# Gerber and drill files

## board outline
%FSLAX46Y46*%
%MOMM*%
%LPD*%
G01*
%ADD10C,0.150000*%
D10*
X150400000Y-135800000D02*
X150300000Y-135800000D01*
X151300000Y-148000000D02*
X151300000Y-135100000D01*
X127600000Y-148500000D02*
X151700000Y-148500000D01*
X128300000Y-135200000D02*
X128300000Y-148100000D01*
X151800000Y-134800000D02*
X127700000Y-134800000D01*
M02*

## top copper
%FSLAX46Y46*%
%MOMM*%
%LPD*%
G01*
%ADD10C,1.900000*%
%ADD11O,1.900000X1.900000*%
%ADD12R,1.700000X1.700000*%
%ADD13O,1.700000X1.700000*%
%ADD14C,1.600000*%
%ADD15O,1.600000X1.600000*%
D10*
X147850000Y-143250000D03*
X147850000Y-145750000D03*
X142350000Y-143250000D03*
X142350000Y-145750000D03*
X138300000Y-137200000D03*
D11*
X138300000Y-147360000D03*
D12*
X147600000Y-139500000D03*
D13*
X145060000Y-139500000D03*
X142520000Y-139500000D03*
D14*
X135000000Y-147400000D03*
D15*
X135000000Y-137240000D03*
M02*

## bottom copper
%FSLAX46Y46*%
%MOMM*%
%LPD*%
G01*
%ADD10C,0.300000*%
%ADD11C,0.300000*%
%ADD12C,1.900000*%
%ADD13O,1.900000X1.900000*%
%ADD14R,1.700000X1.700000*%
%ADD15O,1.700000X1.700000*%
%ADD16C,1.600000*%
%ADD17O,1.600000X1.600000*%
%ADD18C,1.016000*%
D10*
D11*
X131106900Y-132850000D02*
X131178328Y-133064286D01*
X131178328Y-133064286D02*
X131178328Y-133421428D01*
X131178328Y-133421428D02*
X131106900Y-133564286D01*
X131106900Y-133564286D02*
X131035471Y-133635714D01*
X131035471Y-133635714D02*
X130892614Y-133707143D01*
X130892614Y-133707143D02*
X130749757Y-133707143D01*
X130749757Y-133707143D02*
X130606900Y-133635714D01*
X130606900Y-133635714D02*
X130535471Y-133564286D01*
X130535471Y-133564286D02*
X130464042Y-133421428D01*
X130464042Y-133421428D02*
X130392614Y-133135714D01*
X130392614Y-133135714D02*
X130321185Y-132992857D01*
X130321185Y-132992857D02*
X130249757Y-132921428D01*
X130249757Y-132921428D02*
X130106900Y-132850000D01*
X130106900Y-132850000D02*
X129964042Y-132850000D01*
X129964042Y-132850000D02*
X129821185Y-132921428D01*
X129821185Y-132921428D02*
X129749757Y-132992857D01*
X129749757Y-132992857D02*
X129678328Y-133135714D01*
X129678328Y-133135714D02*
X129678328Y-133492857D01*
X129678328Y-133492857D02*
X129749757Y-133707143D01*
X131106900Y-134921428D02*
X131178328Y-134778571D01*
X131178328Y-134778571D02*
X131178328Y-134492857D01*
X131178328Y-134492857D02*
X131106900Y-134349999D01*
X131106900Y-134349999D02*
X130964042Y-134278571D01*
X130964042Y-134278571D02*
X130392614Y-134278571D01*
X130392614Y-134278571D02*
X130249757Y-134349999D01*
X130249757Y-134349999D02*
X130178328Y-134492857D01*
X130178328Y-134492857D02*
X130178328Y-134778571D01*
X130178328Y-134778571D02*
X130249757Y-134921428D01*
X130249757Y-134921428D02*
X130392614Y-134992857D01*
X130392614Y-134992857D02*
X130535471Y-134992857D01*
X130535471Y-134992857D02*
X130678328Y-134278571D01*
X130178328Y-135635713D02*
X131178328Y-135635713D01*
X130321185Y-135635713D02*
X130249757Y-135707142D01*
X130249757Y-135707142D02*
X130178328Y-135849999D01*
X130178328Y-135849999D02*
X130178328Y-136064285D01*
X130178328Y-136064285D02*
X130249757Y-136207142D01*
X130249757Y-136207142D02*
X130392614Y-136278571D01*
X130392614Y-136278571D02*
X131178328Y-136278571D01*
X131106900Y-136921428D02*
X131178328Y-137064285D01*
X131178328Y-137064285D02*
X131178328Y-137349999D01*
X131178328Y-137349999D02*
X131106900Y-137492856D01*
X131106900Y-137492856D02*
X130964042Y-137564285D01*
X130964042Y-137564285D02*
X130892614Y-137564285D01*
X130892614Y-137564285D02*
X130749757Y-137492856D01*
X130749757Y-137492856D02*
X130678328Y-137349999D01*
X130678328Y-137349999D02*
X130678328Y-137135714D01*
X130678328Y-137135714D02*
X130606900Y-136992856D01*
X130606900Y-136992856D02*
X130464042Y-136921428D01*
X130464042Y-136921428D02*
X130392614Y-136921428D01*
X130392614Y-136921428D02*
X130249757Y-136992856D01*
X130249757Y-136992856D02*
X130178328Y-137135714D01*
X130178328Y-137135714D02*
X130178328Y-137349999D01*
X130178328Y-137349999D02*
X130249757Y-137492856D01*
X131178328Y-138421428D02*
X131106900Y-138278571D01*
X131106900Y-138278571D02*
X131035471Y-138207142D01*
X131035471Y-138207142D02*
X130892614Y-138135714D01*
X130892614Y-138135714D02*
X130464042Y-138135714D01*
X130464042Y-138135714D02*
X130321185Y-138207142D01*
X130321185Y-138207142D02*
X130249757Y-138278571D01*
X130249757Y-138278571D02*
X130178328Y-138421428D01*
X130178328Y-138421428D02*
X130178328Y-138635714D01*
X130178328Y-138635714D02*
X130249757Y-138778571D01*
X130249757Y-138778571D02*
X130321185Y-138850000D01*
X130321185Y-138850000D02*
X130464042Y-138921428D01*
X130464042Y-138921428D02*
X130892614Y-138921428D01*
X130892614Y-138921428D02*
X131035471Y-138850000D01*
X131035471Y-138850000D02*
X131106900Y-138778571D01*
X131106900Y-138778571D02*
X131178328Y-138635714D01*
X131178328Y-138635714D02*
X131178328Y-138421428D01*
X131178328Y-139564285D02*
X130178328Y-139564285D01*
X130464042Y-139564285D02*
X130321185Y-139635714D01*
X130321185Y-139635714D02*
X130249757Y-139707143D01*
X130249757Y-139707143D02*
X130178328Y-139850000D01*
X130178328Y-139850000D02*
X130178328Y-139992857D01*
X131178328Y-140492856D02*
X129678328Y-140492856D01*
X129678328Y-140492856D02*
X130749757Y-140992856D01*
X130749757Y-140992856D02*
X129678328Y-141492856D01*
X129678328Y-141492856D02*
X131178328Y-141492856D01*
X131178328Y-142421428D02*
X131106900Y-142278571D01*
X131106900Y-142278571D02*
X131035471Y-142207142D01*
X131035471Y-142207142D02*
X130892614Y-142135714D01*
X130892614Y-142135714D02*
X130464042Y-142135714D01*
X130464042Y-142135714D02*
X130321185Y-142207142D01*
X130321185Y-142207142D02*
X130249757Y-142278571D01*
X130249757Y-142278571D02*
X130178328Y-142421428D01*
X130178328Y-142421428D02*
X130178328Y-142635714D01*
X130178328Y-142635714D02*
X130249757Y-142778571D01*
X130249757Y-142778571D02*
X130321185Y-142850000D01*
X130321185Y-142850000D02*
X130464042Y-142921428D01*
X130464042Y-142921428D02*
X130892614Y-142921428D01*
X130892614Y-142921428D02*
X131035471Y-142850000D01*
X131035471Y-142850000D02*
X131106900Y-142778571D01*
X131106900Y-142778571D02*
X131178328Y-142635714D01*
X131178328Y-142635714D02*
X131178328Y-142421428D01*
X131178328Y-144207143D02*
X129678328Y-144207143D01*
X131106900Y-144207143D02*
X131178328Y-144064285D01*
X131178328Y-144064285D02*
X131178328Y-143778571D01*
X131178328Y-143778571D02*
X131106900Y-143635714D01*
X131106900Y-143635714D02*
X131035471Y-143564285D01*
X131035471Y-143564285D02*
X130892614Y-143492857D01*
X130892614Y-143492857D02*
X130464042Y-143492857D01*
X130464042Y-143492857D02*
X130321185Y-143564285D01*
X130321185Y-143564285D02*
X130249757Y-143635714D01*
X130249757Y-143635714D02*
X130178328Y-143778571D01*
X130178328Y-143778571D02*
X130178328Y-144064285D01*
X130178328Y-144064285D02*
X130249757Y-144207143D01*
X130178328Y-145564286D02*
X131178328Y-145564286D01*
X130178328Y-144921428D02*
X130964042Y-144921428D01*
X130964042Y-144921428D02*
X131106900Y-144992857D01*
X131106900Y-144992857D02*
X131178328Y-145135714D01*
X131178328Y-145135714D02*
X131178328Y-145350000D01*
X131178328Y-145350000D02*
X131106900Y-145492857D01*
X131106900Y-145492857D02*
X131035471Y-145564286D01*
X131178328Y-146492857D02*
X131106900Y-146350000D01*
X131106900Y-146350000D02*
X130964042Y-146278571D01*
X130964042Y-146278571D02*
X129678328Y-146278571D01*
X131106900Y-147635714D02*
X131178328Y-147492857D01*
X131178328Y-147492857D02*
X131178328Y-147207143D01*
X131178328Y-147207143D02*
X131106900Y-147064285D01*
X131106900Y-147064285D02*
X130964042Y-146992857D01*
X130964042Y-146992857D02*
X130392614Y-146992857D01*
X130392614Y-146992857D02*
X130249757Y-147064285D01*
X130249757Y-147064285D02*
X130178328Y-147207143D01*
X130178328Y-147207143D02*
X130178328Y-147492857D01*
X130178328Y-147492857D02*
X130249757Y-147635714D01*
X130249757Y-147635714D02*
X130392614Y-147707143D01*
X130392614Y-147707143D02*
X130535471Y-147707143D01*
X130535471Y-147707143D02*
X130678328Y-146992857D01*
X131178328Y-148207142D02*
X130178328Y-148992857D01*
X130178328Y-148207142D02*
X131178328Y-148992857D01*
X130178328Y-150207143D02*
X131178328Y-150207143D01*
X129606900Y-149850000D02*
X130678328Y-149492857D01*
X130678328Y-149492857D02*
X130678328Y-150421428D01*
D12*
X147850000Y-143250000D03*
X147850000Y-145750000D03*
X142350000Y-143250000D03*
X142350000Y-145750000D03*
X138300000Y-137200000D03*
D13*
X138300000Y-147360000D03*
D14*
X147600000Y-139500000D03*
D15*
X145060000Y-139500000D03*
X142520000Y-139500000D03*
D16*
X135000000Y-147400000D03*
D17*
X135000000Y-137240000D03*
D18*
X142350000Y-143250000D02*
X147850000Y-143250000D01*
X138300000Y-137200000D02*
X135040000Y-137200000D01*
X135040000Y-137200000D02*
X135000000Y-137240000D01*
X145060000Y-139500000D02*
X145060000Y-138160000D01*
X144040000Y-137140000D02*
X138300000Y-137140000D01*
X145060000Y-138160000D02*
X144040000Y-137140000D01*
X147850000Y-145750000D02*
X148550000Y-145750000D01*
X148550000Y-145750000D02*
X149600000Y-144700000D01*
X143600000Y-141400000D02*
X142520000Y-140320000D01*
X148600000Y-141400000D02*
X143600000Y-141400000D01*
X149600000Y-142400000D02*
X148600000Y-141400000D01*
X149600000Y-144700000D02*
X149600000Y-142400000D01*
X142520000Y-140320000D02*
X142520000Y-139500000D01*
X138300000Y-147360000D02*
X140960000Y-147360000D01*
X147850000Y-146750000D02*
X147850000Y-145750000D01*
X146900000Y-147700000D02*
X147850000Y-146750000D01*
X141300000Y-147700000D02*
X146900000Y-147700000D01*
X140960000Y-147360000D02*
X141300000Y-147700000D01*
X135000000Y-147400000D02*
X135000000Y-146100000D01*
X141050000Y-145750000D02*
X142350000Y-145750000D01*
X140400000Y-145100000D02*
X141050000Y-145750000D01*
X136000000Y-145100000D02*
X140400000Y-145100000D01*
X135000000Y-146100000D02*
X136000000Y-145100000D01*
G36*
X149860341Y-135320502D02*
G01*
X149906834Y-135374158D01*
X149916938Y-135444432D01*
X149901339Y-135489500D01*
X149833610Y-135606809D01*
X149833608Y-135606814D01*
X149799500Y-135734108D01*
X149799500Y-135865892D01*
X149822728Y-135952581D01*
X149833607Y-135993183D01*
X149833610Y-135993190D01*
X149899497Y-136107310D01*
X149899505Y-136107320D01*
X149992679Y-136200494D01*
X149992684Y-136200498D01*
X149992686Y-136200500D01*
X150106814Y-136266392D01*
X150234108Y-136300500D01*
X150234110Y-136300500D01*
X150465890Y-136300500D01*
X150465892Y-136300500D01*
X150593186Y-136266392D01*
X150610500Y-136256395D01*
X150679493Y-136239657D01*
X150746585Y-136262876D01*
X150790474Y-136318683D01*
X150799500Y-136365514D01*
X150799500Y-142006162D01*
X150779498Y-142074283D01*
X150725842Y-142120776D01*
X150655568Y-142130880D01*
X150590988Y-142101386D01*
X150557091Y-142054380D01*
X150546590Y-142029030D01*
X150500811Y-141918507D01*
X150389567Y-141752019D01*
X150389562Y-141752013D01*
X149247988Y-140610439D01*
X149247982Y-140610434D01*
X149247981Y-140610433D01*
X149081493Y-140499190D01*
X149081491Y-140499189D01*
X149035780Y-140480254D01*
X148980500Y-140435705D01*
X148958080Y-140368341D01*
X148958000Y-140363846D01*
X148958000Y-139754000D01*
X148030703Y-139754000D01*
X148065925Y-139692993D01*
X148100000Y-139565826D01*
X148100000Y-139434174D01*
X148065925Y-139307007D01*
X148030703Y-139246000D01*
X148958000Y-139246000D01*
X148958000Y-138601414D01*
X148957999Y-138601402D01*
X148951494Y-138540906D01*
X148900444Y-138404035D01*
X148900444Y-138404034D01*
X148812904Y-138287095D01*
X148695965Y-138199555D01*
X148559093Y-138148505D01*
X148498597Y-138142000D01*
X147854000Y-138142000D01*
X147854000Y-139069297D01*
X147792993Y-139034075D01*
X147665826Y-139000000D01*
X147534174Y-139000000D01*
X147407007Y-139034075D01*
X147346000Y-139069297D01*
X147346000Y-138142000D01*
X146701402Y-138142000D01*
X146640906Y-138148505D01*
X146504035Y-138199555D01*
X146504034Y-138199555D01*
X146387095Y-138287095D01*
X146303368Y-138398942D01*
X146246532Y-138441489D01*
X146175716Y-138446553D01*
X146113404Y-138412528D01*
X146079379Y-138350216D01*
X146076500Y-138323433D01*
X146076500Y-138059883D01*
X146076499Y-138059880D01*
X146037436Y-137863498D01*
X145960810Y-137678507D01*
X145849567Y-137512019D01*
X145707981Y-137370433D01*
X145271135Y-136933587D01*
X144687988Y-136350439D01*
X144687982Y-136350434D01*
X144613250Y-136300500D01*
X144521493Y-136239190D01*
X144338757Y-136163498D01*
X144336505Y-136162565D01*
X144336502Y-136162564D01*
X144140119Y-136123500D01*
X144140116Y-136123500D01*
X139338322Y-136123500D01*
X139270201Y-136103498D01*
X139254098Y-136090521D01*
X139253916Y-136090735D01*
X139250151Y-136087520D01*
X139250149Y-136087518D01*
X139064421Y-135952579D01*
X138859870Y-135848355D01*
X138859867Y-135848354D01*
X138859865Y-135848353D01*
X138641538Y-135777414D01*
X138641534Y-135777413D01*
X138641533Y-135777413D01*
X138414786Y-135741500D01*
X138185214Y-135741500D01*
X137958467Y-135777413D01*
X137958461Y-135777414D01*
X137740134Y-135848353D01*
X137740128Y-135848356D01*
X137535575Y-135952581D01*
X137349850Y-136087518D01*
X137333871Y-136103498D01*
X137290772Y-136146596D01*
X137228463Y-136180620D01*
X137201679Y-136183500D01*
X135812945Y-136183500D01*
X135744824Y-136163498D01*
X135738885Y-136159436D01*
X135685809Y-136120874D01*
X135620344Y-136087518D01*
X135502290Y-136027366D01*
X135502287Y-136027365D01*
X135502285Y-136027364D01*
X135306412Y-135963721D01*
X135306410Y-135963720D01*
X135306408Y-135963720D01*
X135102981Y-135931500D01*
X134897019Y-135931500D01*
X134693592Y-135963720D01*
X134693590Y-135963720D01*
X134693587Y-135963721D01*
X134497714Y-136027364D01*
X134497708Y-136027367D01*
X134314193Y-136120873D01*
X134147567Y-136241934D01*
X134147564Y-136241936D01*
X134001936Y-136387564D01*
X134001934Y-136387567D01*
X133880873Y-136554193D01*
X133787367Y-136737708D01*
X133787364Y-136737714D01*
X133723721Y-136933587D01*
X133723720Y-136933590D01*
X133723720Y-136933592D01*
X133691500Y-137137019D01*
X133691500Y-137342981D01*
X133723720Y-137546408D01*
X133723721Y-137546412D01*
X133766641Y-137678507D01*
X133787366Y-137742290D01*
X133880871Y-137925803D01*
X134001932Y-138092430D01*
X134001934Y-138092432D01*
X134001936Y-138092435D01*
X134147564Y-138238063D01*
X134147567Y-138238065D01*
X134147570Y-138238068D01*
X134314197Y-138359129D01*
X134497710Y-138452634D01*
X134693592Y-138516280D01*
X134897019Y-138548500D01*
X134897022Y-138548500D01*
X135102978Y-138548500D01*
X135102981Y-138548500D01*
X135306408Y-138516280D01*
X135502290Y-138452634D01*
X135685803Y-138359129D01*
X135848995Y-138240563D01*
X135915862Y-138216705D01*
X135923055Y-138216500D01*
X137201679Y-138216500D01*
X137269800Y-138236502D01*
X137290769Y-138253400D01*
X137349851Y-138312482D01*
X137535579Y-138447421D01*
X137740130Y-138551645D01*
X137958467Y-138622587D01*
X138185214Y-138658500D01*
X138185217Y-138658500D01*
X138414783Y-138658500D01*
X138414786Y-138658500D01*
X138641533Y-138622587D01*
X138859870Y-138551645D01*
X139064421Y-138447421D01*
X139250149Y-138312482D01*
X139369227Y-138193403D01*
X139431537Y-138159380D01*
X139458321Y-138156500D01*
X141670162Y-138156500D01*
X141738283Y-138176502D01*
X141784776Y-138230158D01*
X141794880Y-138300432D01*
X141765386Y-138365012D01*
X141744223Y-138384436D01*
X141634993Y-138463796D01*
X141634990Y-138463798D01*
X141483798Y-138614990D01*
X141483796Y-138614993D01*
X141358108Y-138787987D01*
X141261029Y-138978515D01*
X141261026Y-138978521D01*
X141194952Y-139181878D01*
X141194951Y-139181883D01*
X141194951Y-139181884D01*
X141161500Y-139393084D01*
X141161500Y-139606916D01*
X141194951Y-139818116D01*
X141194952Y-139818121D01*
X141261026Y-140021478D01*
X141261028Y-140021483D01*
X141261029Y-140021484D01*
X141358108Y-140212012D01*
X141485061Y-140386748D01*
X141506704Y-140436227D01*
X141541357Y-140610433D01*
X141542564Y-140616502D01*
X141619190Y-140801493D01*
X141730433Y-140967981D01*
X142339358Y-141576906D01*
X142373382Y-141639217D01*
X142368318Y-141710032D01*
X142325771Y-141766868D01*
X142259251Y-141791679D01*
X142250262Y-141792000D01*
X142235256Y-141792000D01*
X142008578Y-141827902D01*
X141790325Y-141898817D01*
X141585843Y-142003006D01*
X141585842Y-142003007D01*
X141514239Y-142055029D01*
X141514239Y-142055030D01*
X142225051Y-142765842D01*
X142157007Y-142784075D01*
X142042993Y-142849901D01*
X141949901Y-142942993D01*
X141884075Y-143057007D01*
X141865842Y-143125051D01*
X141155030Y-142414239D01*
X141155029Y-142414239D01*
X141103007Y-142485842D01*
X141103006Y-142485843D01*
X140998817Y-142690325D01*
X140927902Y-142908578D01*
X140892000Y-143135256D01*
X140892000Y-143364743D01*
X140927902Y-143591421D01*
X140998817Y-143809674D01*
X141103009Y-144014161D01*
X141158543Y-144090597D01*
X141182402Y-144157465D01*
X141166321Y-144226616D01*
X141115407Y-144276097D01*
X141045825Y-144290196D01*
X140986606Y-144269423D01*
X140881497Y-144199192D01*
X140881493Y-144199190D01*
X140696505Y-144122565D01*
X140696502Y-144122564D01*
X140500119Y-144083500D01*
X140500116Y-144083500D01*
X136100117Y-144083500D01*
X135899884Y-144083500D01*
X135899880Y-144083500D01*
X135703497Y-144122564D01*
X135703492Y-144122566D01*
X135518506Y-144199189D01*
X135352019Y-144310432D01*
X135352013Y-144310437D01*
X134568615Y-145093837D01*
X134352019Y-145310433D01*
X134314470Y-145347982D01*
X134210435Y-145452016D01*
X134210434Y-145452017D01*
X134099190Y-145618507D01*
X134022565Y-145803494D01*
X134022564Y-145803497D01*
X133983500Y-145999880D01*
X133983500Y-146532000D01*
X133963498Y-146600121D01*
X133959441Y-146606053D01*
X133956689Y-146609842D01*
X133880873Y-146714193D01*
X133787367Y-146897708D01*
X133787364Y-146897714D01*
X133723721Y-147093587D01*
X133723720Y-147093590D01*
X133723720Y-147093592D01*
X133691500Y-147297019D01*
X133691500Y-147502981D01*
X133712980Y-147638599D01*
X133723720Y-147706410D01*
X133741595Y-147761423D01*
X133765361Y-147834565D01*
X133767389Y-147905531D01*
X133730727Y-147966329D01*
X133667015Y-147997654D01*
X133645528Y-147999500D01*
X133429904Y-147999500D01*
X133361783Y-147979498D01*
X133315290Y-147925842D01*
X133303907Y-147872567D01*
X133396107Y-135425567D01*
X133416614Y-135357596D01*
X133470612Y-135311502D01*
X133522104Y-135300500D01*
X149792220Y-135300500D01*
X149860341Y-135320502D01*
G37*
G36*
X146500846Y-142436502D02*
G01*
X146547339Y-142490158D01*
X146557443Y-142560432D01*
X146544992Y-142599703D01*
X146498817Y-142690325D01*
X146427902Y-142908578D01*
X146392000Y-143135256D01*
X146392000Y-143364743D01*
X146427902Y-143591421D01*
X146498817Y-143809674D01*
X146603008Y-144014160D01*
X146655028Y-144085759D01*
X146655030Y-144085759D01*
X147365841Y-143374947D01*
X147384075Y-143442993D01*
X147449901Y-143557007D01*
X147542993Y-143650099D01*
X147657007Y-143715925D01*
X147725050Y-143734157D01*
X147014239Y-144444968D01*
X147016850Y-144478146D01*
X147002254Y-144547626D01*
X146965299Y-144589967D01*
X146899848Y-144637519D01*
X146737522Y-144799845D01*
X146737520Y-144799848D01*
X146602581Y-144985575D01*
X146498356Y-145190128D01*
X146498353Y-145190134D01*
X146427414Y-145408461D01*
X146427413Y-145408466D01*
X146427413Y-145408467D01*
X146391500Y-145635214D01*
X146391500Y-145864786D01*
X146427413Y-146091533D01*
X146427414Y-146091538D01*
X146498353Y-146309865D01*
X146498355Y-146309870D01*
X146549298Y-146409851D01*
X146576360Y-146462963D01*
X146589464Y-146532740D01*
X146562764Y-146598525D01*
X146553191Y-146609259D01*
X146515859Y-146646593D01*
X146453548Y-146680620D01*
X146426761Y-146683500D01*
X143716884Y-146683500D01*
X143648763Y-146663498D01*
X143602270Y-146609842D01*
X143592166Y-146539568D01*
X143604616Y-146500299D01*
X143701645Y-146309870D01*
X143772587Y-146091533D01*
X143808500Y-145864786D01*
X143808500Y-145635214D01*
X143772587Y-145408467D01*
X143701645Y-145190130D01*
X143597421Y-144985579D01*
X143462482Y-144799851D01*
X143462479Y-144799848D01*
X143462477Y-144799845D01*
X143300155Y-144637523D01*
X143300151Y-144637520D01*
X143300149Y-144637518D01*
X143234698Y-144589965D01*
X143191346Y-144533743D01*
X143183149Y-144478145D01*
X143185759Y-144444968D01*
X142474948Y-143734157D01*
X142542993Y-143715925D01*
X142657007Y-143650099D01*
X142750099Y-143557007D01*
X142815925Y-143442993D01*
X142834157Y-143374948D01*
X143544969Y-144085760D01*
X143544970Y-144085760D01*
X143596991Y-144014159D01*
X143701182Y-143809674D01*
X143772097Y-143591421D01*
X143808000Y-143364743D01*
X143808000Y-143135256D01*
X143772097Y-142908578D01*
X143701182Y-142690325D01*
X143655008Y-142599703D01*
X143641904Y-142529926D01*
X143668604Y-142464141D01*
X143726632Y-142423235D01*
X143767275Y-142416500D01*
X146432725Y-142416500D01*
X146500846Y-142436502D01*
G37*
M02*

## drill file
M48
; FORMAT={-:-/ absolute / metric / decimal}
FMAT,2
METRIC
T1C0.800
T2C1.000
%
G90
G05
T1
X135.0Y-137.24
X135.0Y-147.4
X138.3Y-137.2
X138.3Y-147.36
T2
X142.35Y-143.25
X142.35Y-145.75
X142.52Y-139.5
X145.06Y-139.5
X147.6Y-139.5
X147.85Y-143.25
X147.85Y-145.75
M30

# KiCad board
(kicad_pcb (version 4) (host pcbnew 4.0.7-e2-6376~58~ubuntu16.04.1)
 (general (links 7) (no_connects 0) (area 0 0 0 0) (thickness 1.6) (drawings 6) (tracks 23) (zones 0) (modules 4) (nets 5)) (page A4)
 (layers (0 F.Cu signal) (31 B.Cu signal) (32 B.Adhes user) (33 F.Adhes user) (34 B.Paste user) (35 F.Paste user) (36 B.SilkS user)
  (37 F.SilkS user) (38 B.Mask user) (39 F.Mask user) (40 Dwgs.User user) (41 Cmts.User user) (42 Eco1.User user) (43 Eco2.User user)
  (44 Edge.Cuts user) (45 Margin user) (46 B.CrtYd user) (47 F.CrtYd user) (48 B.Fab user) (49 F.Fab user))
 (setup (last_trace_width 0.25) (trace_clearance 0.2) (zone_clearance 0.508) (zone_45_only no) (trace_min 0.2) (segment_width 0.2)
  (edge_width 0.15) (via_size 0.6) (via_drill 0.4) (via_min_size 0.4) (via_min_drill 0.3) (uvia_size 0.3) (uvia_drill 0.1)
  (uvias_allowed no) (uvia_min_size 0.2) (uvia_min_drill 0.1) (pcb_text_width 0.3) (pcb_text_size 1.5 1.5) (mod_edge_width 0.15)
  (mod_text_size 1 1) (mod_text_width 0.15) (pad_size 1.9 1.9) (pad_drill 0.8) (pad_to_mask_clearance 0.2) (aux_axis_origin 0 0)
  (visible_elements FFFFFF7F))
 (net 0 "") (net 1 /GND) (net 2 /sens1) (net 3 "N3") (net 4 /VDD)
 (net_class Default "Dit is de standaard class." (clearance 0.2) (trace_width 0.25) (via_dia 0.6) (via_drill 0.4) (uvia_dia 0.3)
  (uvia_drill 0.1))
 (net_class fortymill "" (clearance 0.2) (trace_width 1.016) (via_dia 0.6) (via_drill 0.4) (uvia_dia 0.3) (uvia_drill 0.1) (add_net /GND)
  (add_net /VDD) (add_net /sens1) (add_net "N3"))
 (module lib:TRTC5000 (layer F.Cu) (at 145.1 144.5 180)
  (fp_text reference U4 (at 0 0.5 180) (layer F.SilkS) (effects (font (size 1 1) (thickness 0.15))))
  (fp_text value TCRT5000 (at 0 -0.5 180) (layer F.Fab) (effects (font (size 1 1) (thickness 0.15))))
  (pad 2 thru_hole circle (at -2.75 1.25 180) (size 1.9 1.9) (drill 1) (layers *.Cu *.Mask) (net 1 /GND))
  (pad 1 thru_hole circle (at -2.75 -1.25 180) (size 1.9 1.9) (drill 1) (layers *.Cu *.Mask) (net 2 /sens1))
  (pad 4 thru_hole circle (at 2.75 1.25 180) (size 1.9 1.9) (drill 1) (layers *.Cu *.Mask) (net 1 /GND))
  (pad 3 thru_hole circle (at 2.75 -1.25 180) (size 1.9 1.9) (drill 1) (layers *.Cu *.Mask) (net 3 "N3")))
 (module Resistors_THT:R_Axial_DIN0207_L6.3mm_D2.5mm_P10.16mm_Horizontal (layer F.Cu) (at 138.3 137.2 270)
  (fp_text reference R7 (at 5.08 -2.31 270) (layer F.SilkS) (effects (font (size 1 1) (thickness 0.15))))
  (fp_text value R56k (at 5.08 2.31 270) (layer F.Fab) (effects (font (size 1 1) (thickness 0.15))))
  (pad 1 thru_hole circle (at 0 0 270) (size 1.9 1.9) (drill 0.8) (layers *.Cu *.Mask) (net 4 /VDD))
  (pad 2 thru_hole oval (at 10.16 0 270) (size 1.9 1.9) (drill 0.8) (layers *.Cu *.Mask) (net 2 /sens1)))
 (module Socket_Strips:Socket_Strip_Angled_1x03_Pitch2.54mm (layer F.Cu) (at 147.6 139.5 270)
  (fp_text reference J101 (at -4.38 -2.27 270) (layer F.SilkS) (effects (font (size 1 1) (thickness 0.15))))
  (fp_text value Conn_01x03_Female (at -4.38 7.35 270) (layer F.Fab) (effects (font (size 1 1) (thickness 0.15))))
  (pad 1 thru_hole rect (at 0 0 270) (size 1.7 1.7) (drill 1) (layers *.Cu *.Mask) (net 1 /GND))
  (pad 2 thru_hole oval (at 0 2.54 270) (size 1.7 1.7) (drill 1) (layers *.Cu *.Mask) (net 4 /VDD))
  (pad 3 thru_hole oval (at 0 5.08 270) (size 1.7 1.7) (drill 1) (layers *.Cu *.Mask) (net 2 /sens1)))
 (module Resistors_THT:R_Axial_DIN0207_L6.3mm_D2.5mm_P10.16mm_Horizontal (layer F.Cu) (at 135 147.4 90)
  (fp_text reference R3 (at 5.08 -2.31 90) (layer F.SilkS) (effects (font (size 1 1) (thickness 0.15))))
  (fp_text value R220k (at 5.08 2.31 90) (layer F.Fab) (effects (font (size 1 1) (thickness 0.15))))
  (pad 1 thru_hole circle (at 0 0 90) (size 1.6 1.6) (drill 0.8) (layers *.Cu *.Mask) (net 3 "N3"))
  (pad 2 thru_hole oval (at 10.16 0 90) (size 1.6 1.6) (drill 0.8) (layers *.Cu *.Mask) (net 4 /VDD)))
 (gr_line (start 150.4 135.8) (end 150.3 135.8) (angle 90) (layer Edge.Cuts) (width 0.15))
 (gr_line (start 151.3 148) (end 151.3 135.1) (angle 90) (layer Edge.Cuts) (width 0.15))
 (gr_line (start 127.6 148.5) (end 151.7 148.5) (angle 90) (layer Edge.Cuts) (width 0.15))
 (gr_line (start 128.3 135.2) (end 128.3 148.1) (angle 90) (layer Edge.Cuts) (width 0.15))
 (gr_line (start 151.8 134.8) (end 127.7 134.8) (angle 90) (layer Edge.Cuts) (width 0.15))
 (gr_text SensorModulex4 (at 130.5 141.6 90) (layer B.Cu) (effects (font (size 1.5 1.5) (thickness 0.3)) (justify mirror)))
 (segment (start 142.35 143.25) (end 147.85 143.25) (width 1.016) (layer B.Cu) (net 1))
 (segment (start 138.3 137.2) (end 135.04 137.2) (width 1.016) (layer B.Cu) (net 4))
 (segment (start 135.04 137.2) (end 135 137.24) (width 1.016) (layer B.Cu) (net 4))
 (segment (start 145.06 139.5) (end 145.06 138.16) (width 1.016) (layer B.Cu) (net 4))
 (segment (start 144.04 137.14) (end 138.3 137.14) (width 1.016) (layer B.Cu) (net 4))
 (segment (start 145.06 138.16) (end 144.04 137.14) (width 1.016) (layer B.Cu) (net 4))
 (segment (start 147.85 145.75) (end 148.55 145.75) (width 1.016) (layer B.Cu) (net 2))
 (segment (start 148.55 145.75) (end 149.6 144.7) (width 1.016) (layer B.Cu) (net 2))
 (segment (start 143.6 141.4) (end 142.52 140.32) (width 1.016) (layer B.Cu) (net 2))
 (segment (start 148.6 141.4) (end 143.6 141.4) (width 1.016) (layer B.Cu) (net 2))
 (segment (start 149.6 142.4) (end 148.6 141.4) (width 1.016) (layer B.Cu) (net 2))
 (segment (start 149.6 144.7) (end 149.6 142.4) (width 1.016) (layer B.Cu) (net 2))
 (segment (start 142.52 140.32) (end 142.52 139.5) (width 1.016) (layer B.Cu) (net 2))
 (segment (start 138.3 147.36) (end 140.96 147.36) (width 1.016) (layer B.Cu) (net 2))
 (segment (start 147.85 146.75) (end 147.85 145.75) (width 1.016) (layer B.Cu) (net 2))
 (segment (start 146.9 147.7) (end 147.85 146.75) (width 1.016) (layer B.Cu) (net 2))
 (segment (start 141.3 147.7) (end 146.9 147.7) (width 1.016) (layer B.Cu) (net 2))
 (segment (start 140.96 147.36) (end 141.3 147.7) (width 1.016) (layer B.Cu) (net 2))
 (segment (start 135 147.4) (end 135 146.1) (width 1.016) (layer B.Cu) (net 3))
 (segment (start 141.05 145.75) (end 142.35 145.75) (width 1.016) (layer B.Cu) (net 3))
 (segment (start 140.4 145.1) (end 141.05 145.75) (width 1.016) (layer B.Cu) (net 3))
 (segment (start 136 145.1) (end 140.4 145.1) (width 1.016) (layer B.Cu) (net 3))
 (segment (start 135 146.1) (end 136 145.1) (width 1.016) (layer B.Cu) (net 3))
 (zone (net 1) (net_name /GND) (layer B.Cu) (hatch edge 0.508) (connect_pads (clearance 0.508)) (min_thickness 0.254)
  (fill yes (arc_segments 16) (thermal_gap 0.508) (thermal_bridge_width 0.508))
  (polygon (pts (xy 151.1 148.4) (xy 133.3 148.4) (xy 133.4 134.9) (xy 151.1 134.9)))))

